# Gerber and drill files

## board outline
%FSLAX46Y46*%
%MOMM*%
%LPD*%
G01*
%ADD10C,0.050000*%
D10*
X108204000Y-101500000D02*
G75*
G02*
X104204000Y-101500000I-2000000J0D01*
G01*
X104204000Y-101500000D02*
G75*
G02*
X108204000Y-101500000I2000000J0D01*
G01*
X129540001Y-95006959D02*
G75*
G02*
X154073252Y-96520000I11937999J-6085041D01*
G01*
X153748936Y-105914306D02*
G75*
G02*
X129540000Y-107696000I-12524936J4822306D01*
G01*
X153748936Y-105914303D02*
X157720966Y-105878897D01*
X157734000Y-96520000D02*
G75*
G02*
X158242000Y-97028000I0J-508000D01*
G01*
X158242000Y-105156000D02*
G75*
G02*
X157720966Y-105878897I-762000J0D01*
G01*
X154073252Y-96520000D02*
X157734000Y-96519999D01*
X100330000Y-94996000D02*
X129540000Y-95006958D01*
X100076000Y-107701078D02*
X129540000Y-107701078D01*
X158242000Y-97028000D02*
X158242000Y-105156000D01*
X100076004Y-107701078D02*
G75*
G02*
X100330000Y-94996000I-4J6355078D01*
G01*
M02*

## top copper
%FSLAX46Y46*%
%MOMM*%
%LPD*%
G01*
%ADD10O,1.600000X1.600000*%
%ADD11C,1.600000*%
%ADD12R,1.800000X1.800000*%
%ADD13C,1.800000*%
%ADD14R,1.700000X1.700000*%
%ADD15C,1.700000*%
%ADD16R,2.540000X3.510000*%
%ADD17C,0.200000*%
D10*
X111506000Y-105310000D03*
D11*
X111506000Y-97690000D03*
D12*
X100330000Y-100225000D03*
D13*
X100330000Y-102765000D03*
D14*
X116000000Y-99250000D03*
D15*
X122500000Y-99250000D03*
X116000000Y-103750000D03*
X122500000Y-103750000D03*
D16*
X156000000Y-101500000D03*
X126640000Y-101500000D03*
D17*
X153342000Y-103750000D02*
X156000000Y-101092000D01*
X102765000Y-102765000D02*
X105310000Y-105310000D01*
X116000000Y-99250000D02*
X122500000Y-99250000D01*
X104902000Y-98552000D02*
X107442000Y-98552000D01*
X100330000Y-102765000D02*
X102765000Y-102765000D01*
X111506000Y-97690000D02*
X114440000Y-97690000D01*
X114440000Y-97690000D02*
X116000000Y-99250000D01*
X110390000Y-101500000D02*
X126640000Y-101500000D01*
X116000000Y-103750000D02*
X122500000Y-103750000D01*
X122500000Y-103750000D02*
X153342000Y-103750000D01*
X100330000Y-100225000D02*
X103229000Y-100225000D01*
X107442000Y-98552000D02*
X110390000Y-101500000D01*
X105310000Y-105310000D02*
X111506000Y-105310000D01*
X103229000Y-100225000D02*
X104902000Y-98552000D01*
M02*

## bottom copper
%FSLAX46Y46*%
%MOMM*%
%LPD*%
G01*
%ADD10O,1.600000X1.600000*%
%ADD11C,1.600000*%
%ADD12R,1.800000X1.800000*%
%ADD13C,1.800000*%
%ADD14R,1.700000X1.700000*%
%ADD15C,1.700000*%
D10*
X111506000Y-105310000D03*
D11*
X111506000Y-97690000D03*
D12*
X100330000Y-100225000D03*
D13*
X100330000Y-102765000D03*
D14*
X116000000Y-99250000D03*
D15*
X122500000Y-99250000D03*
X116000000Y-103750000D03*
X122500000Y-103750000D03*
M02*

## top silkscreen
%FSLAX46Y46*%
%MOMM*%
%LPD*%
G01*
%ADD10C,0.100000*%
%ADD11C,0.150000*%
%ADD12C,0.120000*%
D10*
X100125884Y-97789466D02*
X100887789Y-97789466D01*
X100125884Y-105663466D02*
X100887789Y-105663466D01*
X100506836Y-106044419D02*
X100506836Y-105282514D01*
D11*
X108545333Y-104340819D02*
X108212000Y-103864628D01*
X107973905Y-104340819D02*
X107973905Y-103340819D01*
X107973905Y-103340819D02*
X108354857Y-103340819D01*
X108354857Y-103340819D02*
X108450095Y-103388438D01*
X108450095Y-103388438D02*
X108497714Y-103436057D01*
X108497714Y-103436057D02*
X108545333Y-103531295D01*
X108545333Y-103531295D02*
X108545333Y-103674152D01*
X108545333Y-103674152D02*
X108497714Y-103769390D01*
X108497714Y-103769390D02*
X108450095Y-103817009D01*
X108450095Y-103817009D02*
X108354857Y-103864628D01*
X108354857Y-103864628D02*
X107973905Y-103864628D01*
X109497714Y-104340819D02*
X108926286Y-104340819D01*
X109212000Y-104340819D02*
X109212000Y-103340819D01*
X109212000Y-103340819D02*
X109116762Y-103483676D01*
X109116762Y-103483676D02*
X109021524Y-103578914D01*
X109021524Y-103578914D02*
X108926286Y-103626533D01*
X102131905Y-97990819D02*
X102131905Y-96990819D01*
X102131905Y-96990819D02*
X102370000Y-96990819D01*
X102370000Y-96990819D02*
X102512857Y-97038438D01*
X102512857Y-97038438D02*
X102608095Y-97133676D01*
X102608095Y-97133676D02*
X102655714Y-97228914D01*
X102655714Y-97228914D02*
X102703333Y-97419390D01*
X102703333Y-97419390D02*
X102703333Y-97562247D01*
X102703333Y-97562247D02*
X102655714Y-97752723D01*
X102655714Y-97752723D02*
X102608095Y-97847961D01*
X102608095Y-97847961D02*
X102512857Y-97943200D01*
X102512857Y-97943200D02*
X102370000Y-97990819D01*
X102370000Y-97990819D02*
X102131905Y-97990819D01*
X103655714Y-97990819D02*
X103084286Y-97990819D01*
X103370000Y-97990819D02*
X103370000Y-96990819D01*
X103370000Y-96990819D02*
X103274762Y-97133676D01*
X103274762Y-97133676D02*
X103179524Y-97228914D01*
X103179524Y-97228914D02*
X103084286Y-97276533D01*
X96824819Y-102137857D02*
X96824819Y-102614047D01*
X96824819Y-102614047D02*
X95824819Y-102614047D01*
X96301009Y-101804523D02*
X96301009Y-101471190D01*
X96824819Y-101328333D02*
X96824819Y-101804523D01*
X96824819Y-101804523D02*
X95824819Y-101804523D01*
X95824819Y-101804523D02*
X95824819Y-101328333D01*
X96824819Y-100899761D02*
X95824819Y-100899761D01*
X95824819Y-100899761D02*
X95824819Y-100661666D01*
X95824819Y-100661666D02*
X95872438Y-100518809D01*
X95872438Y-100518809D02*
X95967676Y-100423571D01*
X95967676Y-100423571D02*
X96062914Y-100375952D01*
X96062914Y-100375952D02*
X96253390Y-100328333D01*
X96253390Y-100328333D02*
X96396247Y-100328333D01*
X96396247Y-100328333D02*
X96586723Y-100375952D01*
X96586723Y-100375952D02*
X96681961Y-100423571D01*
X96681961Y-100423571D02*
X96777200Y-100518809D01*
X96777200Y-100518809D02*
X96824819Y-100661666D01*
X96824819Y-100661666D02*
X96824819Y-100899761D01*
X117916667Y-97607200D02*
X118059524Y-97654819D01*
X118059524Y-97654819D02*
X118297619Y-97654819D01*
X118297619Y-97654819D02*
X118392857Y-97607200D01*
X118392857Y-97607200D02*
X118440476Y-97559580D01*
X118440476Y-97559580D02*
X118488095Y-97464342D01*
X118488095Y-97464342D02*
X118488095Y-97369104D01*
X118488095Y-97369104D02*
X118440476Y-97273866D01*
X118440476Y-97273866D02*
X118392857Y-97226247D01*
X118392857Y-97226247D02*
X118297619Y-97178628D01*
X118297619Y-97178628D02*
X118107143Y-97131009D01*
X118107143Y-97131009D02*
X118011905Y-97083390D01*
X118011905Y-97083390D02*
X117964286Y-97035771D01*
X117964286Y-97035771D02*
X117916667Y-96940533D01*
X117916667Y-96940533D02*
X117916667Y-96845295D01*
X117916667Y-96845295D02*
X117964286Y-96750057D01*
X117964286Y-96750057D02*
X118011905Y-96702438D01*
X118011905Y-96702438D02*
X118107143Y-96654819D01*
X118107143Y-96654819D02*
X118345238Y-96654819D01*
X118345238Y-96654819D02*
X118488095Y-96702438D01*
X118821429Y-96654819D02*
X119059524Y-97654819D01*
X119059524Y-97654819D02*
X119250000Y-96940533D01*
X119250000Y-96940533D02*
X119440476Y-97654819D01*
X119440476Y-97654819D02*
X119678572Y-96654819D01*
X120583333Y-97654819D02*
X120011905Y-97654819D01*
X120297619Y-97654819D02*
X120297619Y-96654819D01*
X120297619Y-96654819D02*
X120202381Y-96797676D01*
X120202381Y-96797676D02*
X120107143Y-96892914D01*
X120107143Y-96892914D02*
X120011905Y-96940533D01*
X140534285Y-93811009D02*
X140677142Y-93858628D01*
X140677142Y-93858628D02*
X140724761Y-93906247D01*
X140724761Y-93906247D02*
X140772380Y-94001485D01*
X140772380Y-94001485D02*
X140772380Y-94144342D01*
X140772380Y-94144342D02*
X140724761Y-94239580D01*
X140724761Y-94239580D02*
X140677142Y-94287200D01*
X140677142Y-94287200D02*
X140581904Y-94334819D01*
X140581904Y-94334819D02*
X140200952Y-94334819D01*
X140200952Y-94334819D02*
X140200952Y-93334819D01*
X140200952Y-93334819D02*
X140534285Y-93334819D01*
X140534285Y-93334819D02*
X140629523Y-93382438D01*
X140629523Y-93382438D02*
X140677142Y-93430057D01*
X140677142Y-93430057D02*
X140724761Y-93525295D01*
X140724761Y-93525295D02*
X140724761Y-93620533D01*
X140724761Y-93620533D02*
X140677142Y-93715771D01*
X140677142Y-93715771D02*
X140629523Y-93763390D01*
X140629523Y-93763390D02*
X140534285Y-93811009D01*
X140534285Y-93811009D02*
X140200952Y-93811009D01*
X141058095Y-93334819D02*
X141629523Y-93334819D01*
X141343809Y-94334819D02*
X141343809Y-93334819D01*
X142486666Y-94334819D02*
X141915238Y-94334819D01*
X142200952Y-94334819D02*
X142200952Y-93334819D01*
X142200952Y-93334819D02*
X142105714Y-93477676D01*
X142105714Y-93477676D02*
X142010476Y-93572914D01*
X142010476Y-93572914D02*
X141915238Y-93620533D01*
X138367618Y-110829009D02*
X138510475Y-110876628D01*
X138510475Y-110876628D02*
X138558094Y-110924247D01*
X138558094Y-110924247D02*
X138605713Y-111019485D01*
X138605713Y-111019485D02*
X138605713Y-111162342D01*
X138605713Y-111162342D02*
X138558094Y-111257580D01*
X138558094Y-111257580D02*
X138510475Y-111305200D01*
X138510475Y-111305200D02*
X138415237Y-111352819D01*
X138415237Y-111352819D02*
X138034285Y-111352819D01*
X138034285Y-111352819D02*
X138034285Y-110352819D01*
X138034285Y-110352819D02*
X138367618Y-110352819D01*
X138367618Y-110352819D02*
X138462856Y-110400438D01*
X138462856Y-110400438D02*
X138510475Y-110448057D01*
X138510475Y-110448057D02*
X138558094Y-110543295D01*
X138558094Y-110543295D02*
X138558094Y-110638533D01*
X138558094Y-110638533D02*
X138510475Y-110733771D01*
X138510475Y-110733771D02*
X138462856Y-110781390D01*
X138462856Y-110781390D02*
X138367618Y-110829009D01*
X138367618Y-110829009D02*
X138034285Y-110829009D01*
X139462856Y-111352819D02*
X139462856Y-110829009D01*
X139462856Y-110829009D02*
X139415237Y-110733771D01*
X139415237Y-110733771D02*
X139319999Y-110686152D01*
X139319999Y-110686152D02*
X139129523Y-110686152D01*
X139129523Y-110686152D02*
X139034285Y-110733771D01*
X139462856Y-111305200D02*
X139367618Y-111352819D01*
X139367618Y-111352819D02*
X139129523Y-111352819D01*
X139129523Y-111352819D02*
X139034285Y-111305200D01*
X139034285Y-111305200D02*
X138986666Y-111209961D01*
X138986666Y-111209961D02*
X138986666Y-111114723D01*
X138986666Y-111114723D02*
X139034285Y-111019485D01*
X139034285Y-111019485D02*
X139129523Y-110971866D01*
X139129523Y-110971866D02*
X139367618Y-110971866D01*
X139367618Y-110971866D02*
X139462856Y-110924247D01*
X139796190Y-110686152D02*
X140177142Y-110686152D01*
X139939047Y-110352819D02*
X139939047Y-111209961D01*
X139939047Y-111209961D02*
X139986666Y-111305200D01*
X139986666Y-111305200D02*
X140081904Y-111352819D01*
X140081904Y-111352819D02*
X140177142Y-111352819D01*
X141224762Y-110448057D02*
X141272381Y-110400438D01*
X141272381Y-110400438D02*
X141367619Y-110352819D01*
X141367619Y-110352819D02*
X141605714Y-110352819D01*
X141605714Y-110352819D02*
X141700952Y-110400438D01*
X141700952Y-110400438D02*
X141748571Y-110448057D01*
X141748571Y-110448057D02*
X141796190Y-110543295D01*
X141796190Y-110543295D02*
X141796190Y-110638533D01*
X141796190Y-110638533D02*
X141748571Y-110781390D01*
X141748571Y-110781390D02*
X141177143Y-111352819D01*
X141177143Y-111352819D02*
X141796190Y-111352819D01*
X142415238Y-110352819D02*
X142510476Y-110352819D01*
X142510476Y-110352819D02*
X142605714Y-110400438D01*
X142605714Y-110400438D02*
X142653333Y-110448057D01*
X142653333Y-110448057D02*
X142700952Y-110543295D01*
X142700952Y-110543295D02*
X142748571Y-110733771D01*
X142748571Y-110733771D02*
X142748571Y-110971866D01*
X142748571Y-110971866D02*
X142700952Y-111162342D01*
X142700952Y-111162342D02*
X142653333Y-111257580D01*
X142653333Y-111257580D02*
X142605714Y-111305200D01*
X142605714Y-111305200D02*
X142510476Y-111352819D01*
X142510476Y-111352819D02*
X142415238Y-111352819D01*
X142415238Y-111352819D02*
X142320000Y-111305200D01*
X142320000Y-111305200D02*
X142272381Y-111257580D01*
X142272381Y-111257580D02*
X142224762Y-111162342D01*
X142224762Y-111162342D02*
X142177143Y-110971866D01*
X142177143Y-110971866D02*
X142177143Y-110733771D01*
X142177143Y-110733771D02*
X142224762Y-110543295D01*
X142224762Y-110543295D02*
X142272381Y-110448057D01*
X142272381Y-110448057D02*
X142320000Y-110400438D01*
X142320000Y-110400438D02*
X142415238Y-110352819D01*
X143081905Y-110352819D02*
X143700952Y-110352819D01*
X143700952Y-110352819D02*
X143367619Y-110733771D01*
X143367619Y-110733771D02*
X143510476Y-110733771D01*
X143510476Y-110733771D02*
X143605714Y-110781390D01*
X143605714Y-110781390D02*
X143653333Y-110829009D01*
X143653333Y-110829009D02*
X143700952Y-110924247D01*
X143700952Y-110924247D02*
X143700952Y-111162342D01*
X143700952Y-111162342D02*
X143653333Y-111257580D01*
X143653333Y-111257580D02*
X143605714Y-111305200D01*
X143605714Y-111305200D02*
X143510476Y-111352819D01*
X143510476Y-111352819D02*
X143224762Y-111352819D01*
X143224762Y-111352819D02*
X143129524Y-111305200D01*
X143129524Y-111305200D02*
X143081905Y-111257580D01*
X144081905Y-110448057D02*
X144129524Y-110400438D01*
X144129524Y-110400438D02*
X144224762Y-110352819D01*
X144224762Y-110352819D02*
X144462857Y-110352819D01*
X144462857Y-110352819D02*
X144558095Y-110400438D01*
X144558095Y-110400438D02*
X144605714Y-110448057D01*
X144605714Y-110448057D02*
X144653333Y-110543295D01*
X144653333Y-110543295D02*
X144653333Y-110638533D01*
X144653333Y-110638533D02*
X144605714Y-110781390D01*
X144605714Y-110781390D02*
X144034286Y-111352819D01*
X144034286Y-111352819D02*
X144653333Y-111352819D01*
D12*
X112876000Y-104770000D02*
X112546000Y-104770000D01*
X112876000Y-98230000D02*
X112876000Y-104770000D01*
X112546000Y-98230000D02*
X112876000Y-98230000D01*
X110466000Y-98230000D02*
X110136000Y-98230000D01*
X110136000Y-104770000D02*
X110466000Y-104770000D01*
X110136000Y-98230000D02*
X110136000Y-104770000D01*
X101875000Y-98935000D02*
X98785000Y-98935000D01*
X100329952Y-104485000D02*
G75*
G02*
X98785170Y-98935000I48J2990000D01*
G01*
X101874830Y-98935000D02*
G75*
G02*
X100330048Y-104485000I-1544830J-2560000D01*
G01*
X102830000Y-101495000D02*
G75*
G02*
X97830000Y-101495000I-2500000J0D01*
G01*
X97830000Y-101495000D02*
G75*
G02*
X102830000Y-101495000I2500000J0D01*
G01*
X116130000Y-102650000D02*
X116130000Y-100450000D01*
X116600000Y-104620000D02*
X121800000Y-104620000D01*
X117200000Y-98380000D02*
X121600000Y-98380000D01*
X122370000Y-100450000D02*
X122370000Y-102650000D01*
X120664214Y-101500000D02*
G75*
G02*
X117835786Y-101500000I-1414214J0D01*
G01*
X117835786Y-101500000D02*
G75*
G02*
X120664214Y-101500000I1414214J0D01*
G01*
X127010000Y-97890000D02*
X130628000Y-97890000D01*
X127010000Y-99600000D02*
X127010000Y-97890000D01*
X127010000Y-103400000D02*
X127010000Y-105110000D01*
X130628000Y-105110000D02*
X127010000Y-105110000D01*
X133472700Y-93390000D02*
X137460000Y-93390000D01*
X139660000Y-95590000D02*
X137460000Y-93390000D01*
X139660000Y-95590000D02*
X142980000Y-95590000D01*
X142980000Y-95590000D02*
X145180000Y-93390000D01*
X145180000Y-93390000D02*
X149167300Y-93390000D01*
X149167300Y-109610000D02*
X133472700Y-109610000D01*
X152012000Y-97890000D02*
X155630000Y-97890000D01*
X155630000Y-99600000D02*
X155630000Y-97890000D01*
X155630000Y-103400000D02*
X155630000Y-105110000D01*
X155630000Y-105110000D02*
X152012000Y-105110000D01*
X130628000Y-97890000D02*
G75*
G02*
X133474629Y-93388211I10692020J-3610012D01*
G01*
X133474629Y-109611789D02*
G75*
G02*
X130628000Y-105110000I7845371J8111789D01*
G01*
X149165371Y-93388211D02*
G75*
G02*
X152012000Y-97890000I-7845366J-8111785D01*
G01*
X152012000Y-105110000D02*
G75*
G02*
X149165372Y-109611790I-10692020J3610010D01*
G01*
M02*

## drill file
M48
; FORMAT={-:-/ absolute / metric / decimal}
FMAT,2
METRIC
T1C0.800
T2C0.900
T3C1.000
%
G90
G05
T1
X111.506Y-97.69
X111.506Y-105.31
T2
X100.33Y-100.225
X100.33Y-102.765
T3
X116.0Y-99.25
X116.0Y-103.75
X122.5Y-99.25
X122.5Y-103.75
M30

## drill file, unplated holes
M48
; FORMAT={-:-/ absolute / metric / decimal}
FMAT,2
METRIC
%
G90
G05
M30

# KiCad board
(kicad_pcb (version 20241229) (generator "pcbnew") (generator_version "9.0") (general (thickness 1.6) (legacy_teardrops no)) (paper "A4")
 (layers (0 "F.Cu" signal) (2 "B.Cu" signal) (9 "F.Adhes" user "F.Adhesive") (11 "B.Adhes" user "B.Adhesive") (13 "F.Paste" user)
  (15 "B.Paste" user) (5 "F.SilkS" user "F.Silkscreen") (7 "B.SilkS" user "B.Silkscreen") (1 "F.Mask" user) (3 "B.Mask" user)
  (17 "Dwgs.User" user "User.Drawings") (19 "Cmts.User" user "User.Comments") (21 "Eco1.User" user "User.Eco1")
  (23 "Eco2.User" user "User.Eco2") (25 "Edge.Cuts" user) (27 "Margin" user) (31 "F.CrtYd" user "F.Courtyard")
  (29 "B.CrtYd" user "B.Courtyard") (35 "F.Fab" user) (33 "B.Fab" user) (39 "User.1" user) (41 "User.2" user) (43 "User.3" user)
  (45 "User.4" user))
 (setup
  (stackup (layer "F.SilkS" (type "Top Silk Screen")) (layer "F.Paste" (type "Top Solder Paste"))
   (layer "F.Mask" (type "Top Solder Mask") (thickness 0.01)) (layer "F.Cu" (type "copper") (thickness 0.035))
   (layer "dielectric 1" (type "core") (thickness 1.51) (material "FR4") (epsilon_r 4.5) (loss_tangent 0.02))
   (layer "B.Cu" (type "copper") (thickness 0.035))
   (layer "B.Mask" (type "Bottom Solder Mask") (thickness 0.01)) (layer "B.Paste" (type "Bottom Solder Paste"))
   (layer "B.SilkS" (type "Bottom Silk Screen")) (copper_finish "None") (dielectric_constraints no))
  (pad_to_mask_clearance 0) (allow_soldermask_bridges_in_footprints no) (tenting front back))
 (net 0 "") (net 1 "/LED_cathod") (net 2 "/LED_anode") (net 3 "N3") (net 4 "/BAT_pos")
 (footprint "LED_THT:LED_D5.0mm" (layer "F.Cu") (at 100.33 100.225 -90)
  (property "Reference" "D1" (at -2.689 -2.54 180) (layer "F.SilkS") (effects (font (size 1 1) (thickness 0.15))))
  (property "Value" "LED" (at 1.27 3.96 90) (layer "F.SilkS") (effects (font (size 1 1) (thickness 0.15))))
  (fp_line (start -1.29 -1.545) (end -1.29 1.545) (stroke (width 0.12) (type solid)) (layer "F.SilkS"))
  (fp_arc (start 4.26 0.000048) (mid 2.071756 2.880501) (end -1.29 1.54483) (stroke (width 0.12) (type solid)) (layer "F.SilkS"))
  (fp_arc (start -1.29 -1.54483) (mid 2.071756 -2.880501) (end 4.26 -0.000048) (stroke (width 0.12) (type solid)) (layer "F.SilkS"))
  (fp_circle (center 1.27 0) (end 3.77 0) (stroke (width 0.12) (type solid)) (fill no) (layer "F.SilkS"))
  (pad "1" thru_hole rect (at 0 0 270) (size 1.8 1.8) (drill 0.9) (layers "*.Cu" "*.Mask") (remove_unused_layers no) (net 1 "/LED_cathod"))
  (pad "2" thru_hole circle (at 2.54 0 270) (size 1.8 1.8) (drill 0.9) (layers "*.Cu" "*.Mask") (remove_unused_layers no)
   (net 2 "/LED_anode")))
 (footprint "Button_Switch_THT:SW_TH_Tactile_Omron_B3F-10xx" (layer "F.Cu") (at 116 99.25)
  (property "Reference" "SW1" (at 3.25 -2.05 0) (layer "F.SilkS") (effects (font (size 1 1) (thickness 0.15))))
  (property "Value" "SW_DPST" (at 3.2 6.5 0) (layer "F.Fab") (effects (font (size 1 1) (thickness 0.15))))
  (fp_line (start 0.13 3.4) (end 0.13 1.2) (stroke (width 0.12) (type solid)) (layer "F.SilkS"))
  (fp_line (start 0.6 5.37) (end 5.8 5.37) (stroke (width 0.12) (type solid)) (layer "F.SilkS"))
  (fp_line (start 1.2 -0.87) (end 5.6 -0.87) (stroke (width 0.12) (type solid)) (layer "F.SilkS"))
  (fp_line (start 6.37 1.2) (end 6.37 3.4) (stroke (width 0.12) (type solid)) (layer "F.SilkS"))
  (fp_circle (center 3.25 2.25) (end 4.25 3.25) (stroke (width 0.12) (type solid)) (fill no) (layer "F.SilkS"))
  (pad "1" thru_hole rect (at 0 0) (size 1.7 1.7) (drill 1) (layers "*.Cu" "*.Mask") (remove_unused_layers no) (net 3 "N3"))
  (pad "1" thru_hole circle (at 6.5 0) (size 1.7 1.7) (drill 1) (layers "*.Cu" "*.Mask") (remove_unused_layers no) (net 3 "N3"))
  (pad "2" thru_hole circle (at 0 4.5) (size 1.7 1.7) (drill 1) (layers "*.Cu" "*.Mask") (remove_unused_layers no) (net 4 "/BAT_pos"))
  (pad "2" thru_hole circle (at 6.5 4.5) (size 1.7 1.7) (drill 1) (layers "*.Cu" "*.Mask") (remove_unused_layers no) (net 4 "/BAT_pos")))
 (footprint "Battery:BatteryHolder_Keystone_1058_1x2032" (layer "F.Cu") (at 141.32 101.5 180)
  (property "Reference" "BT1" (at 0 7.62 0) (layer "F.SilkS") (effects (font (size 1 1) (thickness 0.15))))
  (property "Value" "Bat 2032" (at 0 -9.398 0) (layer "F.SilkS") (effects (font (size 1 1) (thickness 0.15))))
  (fp_line (start 14.31 3.61) (end 10.692 3.61) (stroke (width 0.12) (type solid)) (layer "F.SilkS"))
  (fp_line (start 14.31 1.9) (end 14.31 3.61) (stroke (width 0.12) (type solid)) (layer "F.SilkS"))
  (fp_line (start 14.31 -1.9) (end 14.31 -3.61) (stroke (width 0.12) (type solid)) (layer "F.SilkS"))
  (fp_line (start 10.692 -3.61) (end 14.31 -3.61) (stroke (width 0.12) (type solid)) (layer "F.SilkS"))
  (fp_line (start 7.8473 8.11) (end 3.86 8.11) (stroke (width 0.12) (type solid)) (layer "F.SilkS"))
  (fp_line (start 1.66 5.91) (end 3.86 8.11) (stroke (width 0.12) (type solid)) (layer "F.SilkS"))
  (fp_line (start 1.66 5.91) (end -1.66 5.91) (stroke (width 0.12) (type solid)) (layer "F.SilkS"))
  (fp_line (start -1.66 5.91) (end -3.86 8.11) (stroke (width 0.12) (type solid)) (layer "F.SilkS"))
  (fp_line (start -3.86 8.11) (end -7.8473 8.11) (stroke (width 0.12) (type solid)) (layer "F.SilkS"))
  (fp_line (start -7.8473 -8.11) (end 7.8473 -8.11) (stroke (width 0.12) (type solid)) (layer "F.SilkS"))
  (fp_line (start -10.692 3.61) (end -14.31 3.61) (stroke (width 0.12) (type solid)) (layer "F.SilkS"))
  (fp_line (start -14.31 1.9) (end -14.31 3.61) (stroke (width 0.12) (type solid)) (layer "F.SilkS"))
  (fp_line (start -14.31 -1.9) (end -14.31 -3.61) (stroke (width 0.12) (type solid)) (layer "F.SilkS"))
  (fp_line (start -14.31 -3.61) (end -10.692 -3.61) (stroke (width 0.12) (type solid)) (layer "F.SilkS"))
  (fp_arc (start 10.692 3.61) (mid 9.538084 6.031244) (end 7.845371 8.111789) (stroke (width 0.12) (type solid)) (layer "F.SilkS"))
  (fp_arc (start 7.845371 -8.111789) (mid 9.538085 -6.031244) (end 10.692 -3.61) (stroke (width 0.12) (type solid)) (layer "F.SilkS"))
  (fp_arc (start -7.845371 8.111789) (mid -9.538085 6.031244) (end -10.692 3.61) (stroke (width 0.12) (type solid)) (layer "F.SilkS"))
  (fp_arc (start -10.692 -3.61) (mid -9.538084 -6.031244) (end -7.845371 -8.111789) (stroke (width 0.12) (type solid)) (layer "F.SilkS"))
  (pad "1" smd rect (at -14.68 0 180) (size 2.54 3.51) (layers "F.Cu" "F.Mask" "F.Paste") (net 4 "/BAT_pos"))
  (pad "2" smd rect (at 14.68 0 180) (size 2.54 3.51) (layers "F.Cu" "F.Mask" "F.Paste") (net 1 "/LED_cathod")))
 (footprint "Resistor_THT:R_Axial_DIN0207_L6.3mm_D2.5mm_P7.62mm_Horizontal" (layer "F.Cu") (at 111.506 97.69 -90)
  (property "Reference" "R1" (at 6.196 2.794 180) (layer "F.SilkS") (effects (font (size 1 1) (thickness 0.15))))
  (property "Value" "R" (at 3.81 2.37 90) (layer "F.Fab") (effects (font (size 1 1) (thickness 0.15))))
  (fp_line (start 0.54 1.37) (end 7.08 1.37) (stroke (width 0.12) (type solid)) (layer "F.SilkS"))
  (fp_line (start 7.08 1.37) (end 7.08 1.04) (stroke (width 0.12) (type solid)) (layer "F.SilkS"))
  (fp_line (start 0.54 1.04) (end 0.54 1.37) (stroke (width 0.12) (type solid)) (layer "F.SilkS"))
  (fp_line (start 0.54 -1.04) (end 0.54 -1.37) (stroke (width 0.12) (type solid)) (layer "F.SilkS"))
  (fp_line (start 0.54 -1.37) (end 7.08 -1.37) (stroke (width 0.12) (type solid)) (layer "F.SilkS"))
  (fp_line (start 7.08 -1.37) (end 7.08 -1.04) (stroke (width 0.12) (type solid)) (layer "F.SilkS"))
  (pad "1" thru_hole circle (at 0 0 270) (size 1.6 1.6) (drill 0.8) (layers "*.Cu" "*.Mask") (remove_unused_layers no) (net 3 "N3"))
  (pad "2" thru_hole oval (at 7.62 0 270) (size 1.6 1.6) (drill 0.8) (layers "*.Cu" "*.Mask") (remove_unused_layers no) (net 2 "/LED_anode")))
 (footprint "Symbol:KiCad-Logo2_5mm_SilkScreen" (layer "B.Cu") (at 141.986 100.838 180)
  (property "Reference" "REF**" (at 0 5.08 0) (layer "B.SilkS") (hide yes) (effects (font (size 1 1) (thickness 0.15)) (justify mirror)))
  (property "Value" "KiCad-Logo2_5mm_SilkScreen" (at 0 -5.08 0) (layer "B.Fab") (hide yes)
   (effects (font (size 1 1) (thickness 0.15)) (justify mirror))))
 (gr_arc (start 129.540001 95.006959) (mid 142.302814 87.718024) (end 154.073252 96.52) (stroke (width 0.05) (type default)) (locked yes)
  (layer "Edge.Cuts"))
 (gr_arc (start 153.748936 105.914306) (mid 142.20909 114.477001) (end 129.54 107.696) (stroke (width 0.05) (type default)) (locked yes)
  (layer "Edge.Cuts"))
 (gr_line (start 153.748936 105.914303) (end 157.720966 105.878897) (stroke (width 0.05) (type default)) (locked yes) (layer "Edge.Cuts"))
 (gr_arc (start 157.734 96.52) (mid 158.09321 96.66879) (end 158.242 97.028) (stroke (width 0.05) (type default)) (locked yes)
  (layer "Edge.Cuts"))
 (gr_arc (start 158.242 105.156) (mid 158.098167 105.601549) (end 157.720966 105.878897) (stroke (width 0.05) (type default)) (locked yes)
  (layer "Edge.Cuts"))
 (gr_line (start 154.073252 96.52) (end 157.734 96.519999) (stroke (width 0.05) (type default)) (locked yes) (layer "Edge.Cuts"))
 (gr_line (start 100.33 94.996) (end 129.54 95.006958) (stroke (width 0.05) (type default)) (locked yes) (layer "Edge.Cuts"))
 (gr_line (start 100.076 107.701078) (end 129.54 107.701078) (stroke (width 0.05) (type default)) (locked yes) (layer "Edge.Cuts"))
 (gr_line (start 158.242 97.028) (end 158.242 105.156) (stroke (width 0.05) (type default)) (locked yes) (layer "Edge.Cuts"))
 (gr_arc (start 100.076004 107.701078) (mid 93.722196 101.218977) (end 100.33 94.996) (stroke (width 0.05) (type default)) (locked yes)
  (layer "Edge.Cuts"))
 (gr_circle (center 106.204 101.5) (end 108.204 101.5) (stroke (width 0.05) (type default)) (fill no) (layer "Edge.Cuts"))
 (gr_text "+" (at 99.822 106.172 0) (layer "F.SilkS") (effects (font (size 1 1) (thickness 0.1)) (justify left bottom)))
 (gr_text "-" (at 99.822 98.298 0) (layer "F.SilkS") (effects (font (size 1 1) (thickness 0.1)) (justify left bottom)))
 (segment (start 110.39 101.5) (end 126.64 101.5) (width 0.2) (layer "F.Cu") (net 1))
 (segment (start 104.902 98.552) (end 107.442 98.552) (width 0.2) (layer "F.Cu") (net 1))
 (segment (start 107.442 98.552) (end 110.39 101.5) (width 0.2) (layer "F.Cu") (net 1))
 (segment (start 103.229 100.225) (end 104.902 98.552) (width 0.2) (layer "F.Cu") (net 1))
 (segment (start 100.33 100.225) (end 103.229 100.225) (width 0.2) (layer "F.Cu") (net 1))
 (segment (start 116 103.75) (end 122.5 103.75) (width 0.2) (layer "F.Cu") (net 4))
 (segment (start 122.5 103.75) (end 153.342 103.75) (width 0.2) (layer "F.Cu") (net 4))
 (segment (start 153.342 103.75) (end 156 101.092) (width 0.2) (layer "F.Cu") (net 4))
 (segment (start 105.31 105.31) (end 111.506 105.31) (width 0.2) (layer "F.Cu") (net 2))
 (segment (start 100.33 102.765) (end 102.765 102.765) (width 0.2) (layer "F.Cu") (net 2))
 (segment (start 102.765 102.765) (end 105.31 105.31) (width 0.2) (layer "F.Cu") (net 2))
 (segment (start 116 99.25) (end 122.5 99.25) (width 0.2) (layer "F.Cu") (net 3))
 (segment (start 111.506 97.69) (end 114.44 97.69) (width 0.2) (layer "F.Cu") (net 3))
 (segment (start 114.44 97.69) (end 116 99.25) (width 0.2) (layer "F.Cu") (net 3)))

